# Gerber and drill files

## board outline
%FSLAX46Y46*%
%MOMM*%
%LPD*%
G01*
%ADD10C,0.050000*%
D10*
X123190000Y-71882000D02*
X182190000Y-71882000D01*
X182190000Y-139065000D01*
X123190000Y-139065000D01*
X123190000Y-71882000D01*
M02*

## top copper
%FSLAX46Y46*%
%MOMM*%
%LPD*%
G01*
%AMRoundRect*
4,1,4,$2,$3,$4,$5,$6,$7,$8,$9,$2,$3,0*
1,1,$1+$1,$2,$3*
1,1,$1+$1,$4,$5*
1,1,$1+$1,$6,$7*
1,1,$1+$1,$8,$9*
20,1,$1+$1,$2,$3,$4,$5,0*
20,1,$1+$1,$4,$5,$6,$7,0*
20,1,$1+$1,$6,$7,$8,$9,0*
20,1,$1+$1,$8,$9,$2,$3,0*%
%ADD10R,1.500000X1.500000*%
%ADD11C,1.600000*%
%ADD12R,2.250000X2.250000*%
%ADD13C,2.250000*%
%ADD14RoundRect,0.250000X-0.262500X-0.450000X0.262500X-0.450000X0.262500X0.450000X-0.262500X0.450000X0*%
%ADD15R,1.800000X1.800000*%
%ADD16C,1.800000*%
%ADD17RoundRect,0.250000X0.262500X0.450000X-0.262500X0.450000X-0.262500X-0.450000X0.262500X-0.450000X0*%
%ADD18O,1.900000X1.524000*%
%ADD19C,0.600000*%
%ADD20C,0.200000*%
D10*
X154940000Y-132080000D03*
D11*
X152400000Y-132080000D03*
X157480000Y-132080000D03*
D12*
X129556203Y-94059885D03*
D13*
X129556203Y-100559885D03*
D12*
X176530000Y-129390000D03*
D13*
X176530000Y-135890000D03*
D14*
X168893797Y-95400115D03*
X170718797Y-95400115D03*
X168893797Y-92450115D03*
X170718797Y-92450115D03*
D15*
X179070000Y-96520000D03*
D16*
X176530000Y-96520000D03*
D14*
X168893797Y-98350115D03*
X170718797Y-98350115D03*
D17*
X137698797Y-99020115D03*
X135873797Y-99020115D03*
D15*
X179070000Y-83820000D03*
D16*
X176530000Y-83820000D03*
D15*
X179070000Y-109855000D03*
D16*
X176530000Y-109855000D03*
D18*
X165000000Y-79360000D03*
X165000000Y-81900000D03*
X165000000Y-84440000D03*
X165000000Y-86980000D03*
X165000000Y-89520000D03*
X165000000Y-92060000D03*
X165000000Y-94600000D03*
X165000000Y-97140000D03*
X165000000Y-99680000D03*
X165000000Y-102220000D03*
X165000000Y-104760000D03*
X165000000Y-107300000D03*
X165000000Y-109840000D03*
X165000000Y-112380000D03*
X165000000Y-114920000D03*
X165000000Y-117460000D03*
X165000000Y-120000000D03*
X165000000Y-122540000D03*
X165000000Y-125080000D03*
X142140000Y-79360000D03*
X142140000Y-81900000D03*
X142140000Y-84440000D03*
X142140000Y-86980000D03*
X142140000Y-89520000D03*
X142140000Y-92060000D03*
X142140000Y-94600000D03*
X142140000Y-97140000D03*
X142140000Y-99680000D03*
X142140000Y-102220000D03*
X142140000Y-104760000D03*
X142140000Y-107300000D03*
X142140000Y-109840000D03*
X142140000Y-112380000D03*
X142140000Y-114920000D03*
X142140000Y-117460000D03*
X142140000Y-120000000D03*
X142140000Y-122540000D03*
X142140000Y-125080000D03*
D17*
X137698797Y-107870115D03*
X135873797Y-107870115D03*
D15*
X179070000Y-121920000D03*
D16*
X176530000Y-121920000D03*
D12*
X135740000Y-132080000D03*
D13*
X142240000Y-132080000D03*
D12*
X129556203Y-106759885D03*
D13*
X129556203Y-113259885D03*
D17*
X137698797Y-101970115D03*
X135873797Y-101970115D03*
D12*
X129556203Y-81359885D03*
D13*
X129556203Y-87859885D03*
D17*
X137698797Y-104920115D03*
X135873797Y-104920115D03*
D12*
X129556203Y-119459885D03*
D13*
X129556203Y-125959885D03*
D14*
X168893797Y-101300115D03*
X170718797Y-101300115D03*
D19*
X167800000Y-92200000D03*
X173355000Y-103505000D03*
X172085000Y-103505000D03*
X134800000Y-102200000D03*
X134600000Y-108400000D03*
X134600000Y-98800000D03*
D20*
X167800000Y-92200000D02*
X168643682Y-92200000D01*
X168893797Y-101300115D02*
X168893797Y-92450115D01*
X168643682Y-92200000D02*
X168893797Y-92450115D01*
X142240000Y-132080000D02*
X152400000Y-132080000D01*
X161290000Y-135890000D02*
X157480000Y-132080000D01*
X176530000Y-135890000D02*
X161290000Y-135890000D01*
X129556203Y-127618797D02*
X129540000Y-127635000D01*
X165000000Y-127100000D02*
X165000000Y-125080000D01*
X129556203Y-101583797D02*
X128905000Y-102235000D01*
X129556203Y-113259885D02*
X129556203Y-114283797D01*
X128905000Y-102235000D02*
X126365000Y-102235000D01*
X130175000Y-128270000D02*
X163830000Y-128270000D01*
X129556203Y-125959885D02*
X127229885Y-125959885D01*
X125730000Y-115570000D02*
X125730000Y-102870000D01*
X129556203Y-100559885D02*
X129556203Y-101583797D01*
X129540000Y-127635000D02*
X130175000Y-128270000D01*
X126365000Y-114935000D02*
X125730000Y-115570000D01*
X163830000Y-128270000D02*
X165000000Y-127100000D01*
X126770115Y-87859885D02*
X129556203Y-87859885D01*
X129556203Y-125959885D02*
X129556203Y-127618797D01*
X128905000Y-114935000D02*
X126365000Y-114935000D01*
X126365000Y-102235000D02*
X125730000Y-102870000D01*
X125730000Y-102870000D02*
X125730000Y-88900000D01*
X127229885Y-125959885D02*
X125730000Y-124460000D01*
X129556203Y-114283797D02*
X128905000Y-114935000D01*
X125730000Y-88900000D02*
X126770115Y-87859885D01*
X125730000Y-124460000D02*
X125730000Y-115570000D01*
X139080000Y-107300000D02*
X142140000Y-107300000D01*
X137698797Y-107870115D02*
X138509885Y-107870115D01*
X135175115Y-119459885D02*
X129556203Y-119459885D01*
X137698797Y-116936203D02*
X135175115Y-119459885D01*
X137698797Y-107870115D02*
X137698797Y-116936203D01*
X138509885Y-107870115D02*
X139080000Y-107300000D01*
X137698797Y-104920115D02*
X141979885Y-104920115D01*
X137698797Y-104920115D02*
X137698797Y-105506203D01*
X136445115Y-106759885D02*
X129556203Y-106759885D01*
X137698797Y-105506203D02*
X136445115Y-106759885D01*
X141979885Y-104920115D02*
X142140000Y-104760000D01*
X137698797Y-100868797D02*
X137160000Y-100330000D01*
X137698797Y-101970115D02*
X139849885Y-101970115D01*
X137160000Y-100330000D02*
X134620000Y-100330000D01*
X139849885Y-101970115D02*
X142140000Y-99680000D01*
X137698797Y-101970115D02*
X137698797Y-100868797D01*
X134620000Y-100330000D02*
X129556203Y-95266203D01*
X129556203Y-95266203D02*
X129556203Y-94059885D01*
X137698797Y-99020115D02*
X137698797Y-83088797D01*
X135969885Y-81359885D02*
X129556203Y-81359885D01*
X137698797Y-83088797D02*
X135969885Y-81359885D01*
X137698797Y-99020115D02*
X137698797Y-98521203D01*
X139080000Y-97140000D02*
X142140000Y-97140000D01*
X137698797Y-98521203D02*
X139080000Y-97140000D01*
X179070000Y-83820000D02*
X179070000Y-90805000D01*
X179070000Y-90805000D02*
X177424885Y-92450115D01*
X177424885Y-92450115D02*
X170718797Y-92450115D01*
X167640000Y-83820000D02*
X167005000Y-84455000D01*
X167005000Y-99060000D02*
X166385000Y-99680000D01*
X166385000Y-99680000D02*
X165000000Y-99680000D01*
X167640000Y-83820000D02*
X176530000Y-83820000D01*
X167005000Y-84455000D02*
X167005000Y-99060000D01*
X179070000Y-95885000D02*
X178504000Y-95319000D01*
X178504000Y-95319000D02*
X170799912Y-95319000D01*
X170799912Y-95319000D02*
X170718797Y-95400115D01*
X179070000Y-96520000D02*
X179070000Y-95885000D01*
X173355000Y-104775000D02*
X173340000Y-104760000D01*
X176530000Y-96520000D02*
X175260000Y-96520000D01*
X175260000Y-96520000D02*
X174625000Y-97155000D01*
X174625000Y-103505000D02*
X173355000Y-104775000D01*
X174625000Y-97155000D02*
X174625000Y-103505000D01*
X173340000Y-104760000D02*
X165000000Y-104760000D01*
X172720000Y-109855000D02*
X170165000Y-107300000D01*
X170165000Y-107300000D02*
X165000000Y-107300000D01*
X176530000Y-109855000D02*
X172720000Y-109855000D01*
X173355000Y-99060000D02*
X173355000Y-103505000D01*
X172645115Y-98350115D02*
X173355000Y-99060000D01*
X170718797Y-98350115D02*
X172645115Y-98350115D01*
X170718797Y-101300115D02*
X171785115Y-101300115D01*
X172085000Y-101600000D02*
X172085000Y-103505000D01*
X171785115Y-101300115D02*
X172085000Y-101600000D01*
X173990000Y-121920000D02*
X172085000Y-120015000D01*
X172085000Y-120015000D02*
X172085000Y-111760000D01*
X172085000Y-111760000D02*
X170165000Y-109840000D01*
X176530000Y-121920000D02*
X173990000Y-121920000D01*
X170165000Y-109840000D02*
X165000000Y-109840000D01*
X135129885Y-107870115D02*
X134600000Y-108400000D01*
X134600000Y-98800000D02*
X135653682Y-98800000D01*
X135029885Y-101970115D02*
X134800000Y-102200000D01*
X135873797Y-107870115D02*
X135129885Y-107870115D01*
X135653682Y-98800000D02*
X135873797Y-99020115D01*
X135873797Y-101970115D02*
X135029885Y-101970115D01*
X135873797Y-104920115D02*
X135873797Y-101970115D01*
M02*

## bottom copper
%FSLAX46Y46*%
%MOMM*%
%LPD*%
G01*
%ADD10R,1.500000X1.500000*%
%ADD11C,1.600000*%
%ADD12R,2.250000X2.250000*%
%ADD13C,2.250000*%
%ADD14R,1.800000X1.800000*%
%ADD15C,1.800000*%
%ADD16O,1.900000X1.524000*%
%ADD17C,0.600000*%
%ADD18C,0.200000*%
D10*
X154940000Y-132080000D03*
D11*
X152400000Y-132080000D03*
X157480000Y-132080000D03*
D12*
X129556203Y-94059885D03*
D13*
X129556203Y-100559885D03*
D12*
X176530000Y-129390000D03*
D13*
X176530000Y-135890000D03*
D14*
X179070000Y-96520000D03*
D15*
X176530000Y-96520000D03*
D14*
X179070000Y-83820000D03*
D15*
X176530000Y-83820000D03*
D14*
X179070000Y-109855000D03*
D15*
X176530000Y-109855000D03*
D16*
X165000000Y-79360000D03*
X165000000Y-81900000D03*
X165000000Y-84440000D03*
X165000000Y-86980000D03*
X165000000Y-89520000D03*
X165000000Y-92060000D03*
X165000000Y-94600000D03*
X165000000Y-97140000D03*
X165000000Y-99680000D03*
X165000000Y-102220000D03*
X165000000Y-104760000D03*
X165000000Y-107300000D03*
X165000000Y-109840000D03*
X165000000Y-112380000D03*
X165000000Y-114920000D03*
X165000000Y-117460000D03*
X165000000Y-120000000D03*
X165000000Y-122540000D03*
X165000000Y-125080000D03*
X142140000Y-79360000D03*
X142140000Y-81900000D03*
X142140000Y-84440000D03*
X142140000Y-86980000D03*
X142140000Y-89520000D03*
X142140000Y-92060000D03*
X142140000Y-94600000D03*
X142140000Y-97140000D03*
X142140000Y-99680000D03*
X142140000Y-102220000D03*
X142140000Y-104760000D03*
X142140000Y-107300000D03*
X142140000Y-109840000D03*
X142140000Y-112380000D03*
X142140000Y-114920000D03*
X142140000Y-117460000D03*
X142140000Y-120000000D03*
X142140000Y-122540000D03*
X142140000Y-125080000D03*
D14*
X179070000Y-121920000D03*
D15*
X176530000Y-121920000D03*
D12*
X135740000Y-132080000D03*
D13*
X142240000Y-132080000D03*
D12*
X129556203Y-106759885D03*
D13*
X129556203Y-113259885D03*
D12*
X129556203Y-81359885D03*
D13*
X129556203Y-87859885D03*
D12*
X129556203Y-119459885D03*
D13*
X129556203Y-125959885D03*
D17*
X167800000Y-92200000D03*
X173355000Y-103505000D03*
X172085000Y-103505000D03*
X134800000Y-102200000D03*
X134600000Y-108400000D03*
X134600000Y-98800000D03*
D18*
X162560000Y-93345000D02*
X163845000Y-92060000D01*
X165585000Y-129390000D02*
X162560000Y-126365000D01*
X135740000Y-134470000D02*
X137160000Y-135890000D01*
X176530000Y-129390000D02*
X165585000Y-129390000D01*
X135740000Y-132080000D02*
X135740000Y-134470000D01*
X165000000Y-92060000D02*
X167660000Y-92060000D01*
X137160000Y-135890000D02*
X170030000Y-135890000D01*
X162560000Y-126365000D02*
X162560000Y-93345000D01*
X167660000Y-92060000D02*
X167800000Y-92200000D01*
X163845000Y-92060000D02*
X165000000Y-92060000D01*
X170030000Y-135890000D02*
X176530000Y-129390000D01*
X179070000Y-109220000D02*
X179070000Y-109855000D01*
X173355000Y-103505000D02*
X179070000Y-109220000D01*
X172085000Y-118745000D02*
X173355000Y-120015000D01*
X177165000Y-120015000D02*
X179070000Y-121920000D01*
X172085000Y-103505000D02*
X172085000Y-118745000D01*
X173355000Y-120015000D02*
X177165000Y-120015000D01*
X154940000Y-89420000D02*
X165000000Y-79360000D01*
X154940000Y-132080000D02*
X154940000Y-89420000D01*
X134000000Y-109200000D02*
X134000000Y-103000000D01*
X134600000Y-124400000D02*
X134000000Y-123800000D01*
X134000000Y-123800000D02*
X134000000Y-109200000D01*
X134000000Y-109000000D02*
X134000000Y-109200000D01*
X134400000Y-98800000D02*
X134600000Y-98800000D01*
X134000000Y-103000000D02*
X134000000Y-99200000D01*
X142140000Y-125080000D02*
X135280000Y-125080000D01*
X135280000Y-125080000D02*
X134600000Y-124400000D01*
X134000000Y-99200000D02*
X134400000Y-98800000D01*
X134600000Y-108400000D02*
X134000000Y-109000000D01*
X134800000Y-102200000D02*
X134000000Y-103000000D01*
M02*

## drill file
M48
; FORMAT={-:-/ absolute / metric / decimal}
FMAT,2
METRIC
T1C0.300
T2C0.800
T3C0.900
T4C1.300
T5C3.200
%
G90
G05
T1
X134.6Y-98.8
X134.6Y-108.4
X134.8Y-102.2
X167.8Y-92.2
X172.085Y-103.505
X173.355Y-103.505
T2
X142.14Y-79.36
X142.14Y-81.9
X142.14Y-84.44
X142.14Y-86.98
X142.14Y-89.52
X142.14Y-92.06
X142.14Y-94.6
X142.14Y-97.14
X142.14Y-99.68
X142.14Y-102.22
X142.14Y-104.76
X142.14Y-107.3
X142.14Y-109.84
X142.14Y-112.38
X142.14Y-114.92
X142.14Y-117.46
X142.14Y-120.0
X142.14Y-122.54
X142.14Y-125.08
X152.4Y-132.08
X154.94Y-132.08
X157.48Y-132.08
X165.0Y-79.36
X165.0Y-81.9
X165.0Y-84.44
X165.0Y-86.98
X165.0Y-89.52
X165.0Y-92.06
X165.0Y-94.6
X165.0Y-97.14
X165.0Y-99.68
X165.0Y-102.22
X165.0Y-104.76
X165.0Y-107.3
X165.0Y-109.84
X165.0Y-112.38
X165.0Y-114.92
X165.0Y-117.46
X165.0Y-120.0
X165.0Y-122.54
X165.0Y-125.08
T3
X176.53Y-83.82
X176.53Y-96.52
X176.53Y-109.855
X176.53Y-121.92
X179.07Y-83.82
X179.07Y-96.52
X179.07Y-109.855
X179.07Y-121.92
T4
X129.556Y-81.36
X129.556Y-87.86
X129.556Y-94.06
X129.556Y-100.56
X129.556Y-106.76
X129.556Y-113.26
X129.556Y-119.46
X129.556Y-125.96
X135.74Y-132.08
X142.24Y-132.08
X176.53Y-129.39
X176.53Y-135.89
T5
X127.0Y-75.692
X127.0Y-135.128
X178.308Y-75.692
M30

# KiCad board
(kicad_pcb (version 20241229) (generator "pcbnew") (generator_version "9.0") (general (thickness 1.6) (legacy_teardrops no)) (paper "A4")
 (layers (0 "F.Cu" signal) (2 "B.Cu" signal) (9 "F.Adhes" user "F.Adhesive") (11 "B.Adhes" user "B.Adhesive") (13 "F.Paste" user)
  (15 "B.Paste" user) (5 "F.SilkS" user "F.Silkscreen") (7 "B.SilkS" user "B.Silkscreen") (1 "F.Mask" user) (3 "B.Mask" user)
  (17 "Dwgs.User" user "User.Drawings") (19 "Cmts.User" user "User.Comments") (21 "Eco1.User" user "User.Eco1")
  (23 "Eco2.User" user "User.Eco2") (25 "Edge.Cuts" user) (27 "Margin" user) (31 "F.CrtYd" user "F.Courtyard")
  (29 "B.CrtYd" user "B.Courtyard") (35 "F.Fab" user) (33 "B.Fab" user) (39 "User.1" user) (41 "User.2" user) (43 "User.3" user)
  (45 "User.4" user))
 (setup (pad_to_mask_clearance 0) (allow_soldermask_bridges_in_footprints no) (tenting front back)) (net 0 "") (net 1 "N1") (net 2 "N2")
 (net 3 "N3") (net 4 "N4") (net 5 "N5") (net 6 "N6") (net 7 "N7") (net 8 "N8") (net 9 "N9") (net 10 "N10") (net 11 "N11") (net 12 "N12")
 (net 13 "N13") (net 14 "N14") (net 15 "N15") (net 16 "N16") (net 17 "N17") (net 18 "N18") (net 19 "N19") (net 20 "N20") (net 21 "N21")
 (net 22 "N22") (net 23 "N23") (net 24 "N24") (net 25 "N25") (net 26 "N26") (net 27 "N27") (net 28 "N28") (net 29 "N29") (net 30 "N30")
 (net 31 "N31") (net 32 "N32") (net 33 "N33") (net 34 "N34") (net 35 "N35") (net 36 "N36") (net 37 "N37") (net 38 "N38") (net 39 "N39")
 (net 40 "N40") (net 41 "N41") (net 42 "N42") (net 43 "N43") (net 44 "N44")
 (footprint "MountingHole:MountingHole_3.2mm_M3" (layer "F.Cu") (at 178.308 75.692)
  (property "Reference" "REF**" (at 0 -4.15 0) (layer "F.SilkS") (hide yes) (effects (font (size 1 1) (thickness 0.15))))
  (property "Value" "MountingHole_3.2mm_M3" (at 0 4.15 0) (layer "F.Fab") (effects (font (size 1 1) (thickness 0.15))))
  (pad "" np_thru_hole circle (at 0 0) (size 3.2 3.2) (drill 3.2) (layers "*.Cu" "*.Mask")))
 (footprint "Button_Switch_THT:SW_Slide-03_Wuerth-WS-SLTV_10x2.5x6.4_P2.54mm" (layer "F.Cu") (at 154.94 132.08)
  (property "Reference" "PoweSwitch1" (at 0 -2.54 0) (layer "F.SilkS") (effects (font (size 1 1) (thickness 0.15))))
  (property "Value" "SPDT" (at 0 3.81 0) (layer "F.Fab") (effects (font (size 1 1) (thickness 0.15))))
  (pad "1" thru_hole rect (at 0 0) (size 1.5 1.5) (drill 0.8) (layers "*.Cu" "*.Mask") (remove_unused_layers no) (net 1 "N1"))
  (pad "2" thru_hole circle (at -2.54 0) (size 1.6 1.6) (drill 0.8) (layers "*.Cu" "*.Mask") (remove_unused_layers no) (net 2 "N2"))
  (pad "3" thru_hole circle (at 2.54 0) (size 1.6 1.6) (drill 0.8) (layers "*.Cu" "*.Mask") (remove_unused_layers no) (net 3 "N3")))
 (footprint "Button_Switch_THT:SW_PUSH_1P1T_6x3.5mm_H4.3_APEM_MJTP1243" (layer "F.Cu") (at 129.556203 94.059885 -90)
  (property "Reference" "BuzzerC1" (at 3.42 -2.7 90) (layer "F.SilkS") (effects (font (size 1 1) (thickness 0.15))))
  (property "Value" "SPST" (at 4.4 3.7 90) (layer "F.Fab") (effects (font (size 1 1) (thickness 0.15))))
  (pad "1" thru_hole rect (at 0 0) (size 2.25 2.25) (drill 1.3) (layers "*.Cu" "*.Mask") (remove_unused_layers no) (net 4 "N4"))
  (pad "2" thru_hole circle (at 6.5 0) (size 2.25 2.25) (drill 1.3) (layers "*.Cu" "*.Mask") (remove_unused_layers no) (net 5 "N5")))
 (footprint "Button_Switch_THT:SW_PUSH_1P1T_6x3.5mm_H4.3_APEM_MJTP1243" (layer "F.Cu") (at 176.53 129.39 -90)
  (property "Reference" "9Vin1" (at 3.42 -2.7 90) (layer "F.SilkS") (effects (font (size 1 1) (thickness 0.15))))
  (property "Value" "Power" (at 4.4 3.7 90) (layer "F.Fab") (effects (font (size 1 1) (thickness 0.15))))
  (pad "1" thru_hole rect (at 0 0) (size 2.25 2.25) (drill 1.3) (layers "*.Cu" "*.Mask") (remove_unused_layers no) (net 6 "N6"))
  (pad "2" thru_hole circle (at 6.5 0) (size 2.25 2.25) (drill 1.3) (layers "*.Cu" "*.Mask") (remove_unused_layers no) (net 3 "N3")))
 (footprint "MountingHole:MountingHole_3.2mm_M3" (layer "F.Cu") (at 127 135.128)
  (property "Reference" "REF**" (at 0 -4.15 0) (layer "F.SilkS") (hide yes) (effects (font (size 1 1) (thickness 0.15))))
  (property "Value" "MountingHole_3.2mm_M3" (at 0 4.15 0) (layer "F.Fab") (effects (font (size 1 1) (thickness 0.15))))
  (pad "" np_thru_hole circle (at 0 0) (size 3.2 3.2) (drill 3.2) (layers "*.Cu" "*.Mask")))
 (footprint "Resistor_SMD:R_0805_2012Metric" (layer "F.Cu") (at 169.806297 95.400115)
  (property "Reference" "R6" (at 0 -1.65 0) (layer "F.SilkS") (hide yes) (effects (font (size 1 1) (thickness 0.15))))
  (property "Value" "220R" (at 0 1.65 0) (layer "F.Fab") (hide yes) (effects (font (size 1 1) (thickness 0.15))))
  (pad "1" smd roundrect (at -0.9125 0) (size 1.025 1.4) (layers "F.Cu" "F.Mask" "F.Paste") (roundrect_rratio 0.243902) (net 6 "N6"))
  (pad "2" smd roundrect (at 0.9125 0) (size 1.025 1.4) (layers "F.Cu" "F.Mask" "F.Paste") (roundrect_rratio 0.243902) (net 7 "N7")))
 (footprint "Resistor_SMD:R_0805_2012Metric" (layer "F.Cu") (at 169.806297 92.450115)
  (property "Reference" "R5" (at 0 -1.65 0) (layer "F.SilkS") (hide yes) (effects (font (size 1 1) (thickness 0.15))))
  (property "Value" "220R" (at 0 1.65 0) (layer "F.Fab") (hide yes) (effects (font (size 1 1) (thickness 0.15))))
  (pad "1" smd roundrect (at -0.9125 0) (size 1.025 1.4) (layers "F.Cu" "F.Mask" "F.Paste") (roundrect_rratio 0.243902) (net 6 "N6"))
  (pad "2" smd roundrect (at 0.9125 0) (size 1.025 1.4) (layers "F.Cu" "F.Mask" "F.Paste") (roundrect_rratio 0.243902) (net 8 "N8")))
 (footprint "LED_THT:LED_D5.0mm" (layer "F.Cu") (at 179.07 96.52 180)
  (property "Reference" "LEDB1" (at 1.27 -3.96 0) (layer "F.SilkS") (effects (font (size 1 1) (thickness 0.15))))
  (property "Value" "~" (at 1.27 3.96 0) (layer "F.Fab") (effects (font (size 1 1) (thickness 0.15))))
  (pad "1" thru_hole rect (at 0 0 180) (size 1.8 1.8) (drill 0.9) (layers "*.Cu" "*.Mask") (remove_unused_layers no) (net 7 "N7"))
  (pad "2" thru_hole circle (at 2.54 0 180) (size 1.8 1.8) (drill 0.9) (layers "*.Cu" "*.Mask") (remove_unused_layers no) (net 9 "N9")))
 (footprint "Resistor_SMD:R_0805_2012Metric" (layer "F.Cu") (at 169.806297 98.350115)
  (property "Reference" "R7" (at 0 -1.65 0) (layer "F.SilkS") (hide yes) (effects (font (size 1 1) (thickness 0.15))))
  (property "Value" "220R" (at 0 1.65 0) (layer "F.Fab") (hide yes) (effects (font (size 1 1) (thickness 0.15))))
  (pad "1" smd roundrect (at -0.9125 0) (size 1.025 1.4) (layers "F.Cu" "F.Mask" "F.Paste") (roundrect_rratio 0.243902) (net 6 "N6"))
  (pad "2" smd roundrect (at 0.9125 0) (size 1.025 1.4) (layers "F.Cu" "F.Mask" "F.Paste") (roundrect_rratio 0.243902) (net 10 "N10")))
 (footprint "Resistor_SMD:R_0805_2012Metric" (layer "F.Cu") (at 136.786297 99.020115 180)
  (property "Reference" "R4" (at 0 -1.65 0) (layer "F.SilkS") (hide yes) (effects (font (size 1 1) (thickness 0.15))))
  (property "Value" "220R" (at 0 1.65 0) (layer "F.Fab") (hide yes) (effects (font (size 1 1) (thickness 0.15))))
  (pad "1" smd roundrect (at -0.9125 0 180) (size 1.025 1.4) (layers "F.Cu" "F.Mask" "F.Paste") (roundrect_rratio 0.243902) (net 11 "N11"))
  (pad "2" smd roundrect (at 0.9125 0 180) (size 1.025 1.4) (layers "F.Cu" "F.Mask" "F.Paste") (roundrect_rratio 0.243902) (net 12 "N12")))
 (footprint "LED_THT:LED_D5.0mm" (layer "F.Cu") (at 179.07 83.82 180)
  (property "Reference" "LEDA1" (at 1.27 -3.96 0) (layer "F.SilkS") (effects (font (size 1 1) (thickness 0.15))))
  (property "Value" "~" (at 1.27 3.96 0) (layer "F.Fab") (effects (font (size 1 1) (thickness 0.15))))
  (pad "1" thru_hole rect (at 0 0 180) (size 1.8 1.8) (drill 0.9) (layers "*.Cu" "*.Mask") (remove_unused_layers no) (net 8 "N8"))
  (pad "2" thru_hole circle (at 2.54 0 180) (size 1.8 1.8) (drill 0.9) (layers "*.Cu" "*.Mask") (remove_unused_layers no) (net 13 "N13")))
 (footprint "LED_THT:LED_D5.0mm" (layer "F.Cu") (at 179.07 109.855 180)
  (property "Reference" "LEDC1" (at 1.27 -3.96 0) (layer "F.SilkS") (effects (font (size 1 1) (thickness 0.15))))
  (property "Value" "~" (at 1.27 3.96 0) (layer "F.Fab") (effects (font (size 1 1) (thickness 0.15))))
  (pad "1" thru_hole rect (at 0 0 180) (size 1.8 1.8) (drill 0.9) (layers "*.Cu" "*.Mask") (remove_unused_layers no) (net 10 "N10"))
  (pad "2" thru_hole circle (at 2.54 0 180) (size 1.8 1.8) (drill 0.9) (layers "*.Cu" "*.Mask") (remove_unused_layers no) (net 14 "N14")))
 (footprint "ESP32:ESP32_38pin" (layer "F.Cu") (at 153.456183 102.385111 180)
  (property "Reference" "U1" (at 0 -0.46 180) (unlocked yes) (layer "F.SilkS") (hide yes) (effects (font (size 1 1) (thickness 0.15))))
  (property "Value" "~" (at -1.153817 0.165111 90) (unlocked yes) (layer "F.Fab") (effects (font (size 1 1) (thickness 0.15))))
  (pad "1" thru_hole oval (at -11.543817 23.025111 90) (size 1.524 1.9) (drill 0.8) (layers "*.Cu" "*.Mask") (remove_unused_layers no)
   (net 1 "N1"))
  (pad "2" thru_hole oval (at -11.543817 20.485111 90) (size 1.524 1.9) (drill 0.8) (layers "*.Cu" "*.Mask") (remove_unused_layers no)
   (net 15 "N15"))
  (pad "3" thru_hole oval (at -11.543817 17.945111 90) (size 1.524 1.9) (drill 0.8) (layers "*.Cu" "*.Mask") (remove_unused_layers no)
   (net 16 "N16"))
  (pad "4" thru_hole oval (at -11.543817 15.405111 90) (size 1.524 1.9) (drill 0.8) (layers "*.Cu" "*.Mask") (remove_unused_layers no)
   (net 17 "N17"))
  (pad "5" thru_hole oval (at -11.543817 12.865111 90) (size 1.524 1.9) (drill 0.8) (layers "*.Cu" "*.Mask") (remove_unused_layers no)
   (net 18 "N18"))
  (pad "6" thru_hole oval (at -11.543817 10.325111 90) (size 1.524 1.9) (drill 0.8) (layers "*.Cu" "*.Mask") (remove_unused_layers no)
   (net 6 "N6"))
  (pad "7" thru_hole oval (at -11.543817 7.785111 90) (size 1.524 1.9) (drill 0.8) (layers "*.Cu" "*.Mask") (remove_unused_layers no)
   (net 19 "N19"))
  (pad "8" thru_hole oval (at -11.543817 5.245111 90) (size 1.524 1.9) (drill 0.8) (layers "*.Cu" "*.Mask") (remove_unused_layers no)
   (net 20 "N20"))
  (pad "9" thru_hole oval (at -11.543817 2.705111 90) (size 1.524 1.9) (drill 0.8) (layers "*.Cu" "*.Mask") (remove_unused_layers no)
   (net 13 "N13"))
  (pad "10" thru_hole oval (at -11.543817 0.165111 90) (size 1.524 1.9) (drill 0.8) (layers "*.Cu" "*.Mask") (remove_unused_layers no)
   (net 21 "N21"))
  (pad "11" thru_hole oval (at -11.543817 -2.374889 90) (size 1.524 1.9) (drill 0.8) (layers "*.Cu" "*.Mask") (remove_unused_layers no)
   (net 9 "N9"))
  (pad "12" thru_hole oval (at -11.543817 -4.914889 90) (size 1.524 1.9) (drill 0.8) (layers "*.Cu" "*.Mask") (remove_unused_layers no)
   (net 14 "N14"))
  (pad "13" thru_hole oval (at -11.543817 -7.454889 90) (size 1.524 1.9) (drill 0.8) (layers "*.Cu" "*.Mask") (remove_unused_layers no)
   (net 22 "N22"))
  (pad "14" thru_hole oval (at -11.543817 -9.994889 90) (size 1.524 1.9) (drill 0.8) (layers "*.Cu" "*.Mask") (remove_unused_layers no)
   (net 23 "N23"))
  (pad "15" thru_hole oval (at -11.543817 -12.534889 90) (size 1.524 1.9) (drill 0.8) (layers "*.Cu" "*.Mask") (remove_unused_layers no)
   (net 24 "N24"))
  (pad "16" thru_hole oval (at -11.543817 -15.074889 90) (size 1.524 1.9) (drill 0.8) (layers "*.Cu" "*.Mask") (remove_unused_layers no)
   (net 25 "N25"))
  (pad "17" thru_hole oval (at -11.543817 -17.614889 90) (size 1.524 1.9) (drill 0.8) (layers "*.Cu" "*.Mask") (remove_unused_layers no)
   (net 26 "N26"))
  (pad "18" thru_hole oval (at -11.543817 -20.154889 90) (size 1.524 1.9) (drill 0.8) (layers "*.Cu" "*.Mask") (remove_unused_layers no)
   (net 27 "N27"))
  (pad "19" thru_hole oval (at -11.543817 -22.694889 90) (size 1.524 1.9) (drill 0.8) (layers "*.Cu" "*.Mask") (remove_unused_layers no)
   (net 5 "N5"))
  (pad "20" thru_hole oval (at 11.316183 23.025111 90) (size 1.524 1.9) (drill 0.8) (layers "*.Cu" "*.Mask") (remove_unused_layers no)
   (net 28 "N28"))
  (pad "21" thru_hole oval (at 11.316183 20.485111 90) (size 1.524 1.9) (drill 0.8) (layers "*.Cu" "*.Mask") (remove_unused_layers no)
   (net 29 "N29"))
  (pad "22" thru_hole oval (at 11.316183 17.945111 90) (size 1.524 1.9) (drill 0.8) (layers "*.Cu" "*.Mask") (remove_unused_layers no)
   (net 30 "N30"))
  (pad "23" thru_hole oval (at 11.316183 15.405111 90) (size 1.524 1.9) (drill 0.8) (layers "*.Cu" "*.Mask") (remove_unused_layers no)
   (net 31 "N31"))
  (pad "24" thru_hole oval (at 11.316183 12.865111 90) (size 1.524 1.9) (drill 0.8) (layers "*.Cu" "*.Mask") (remove_unused_layers no)
   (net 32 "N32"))
  (pad "25" thru_hole oval (at 11.316183 10.325111 90) (size 1.524 1.9) (drill 0.8) (layers "*.Cu" "*.Mask") (remove_unused_layers no)
   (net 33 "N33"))
  (pad "26" thru_hole oval (at 11.316183 7.785111 90) (size 1.524 1.9) (drill 0.8) (layers "*.Cu" "*.Mask") (remove_unused_layers no)
   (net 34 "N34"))
  (pad "27" thru_hole oval (at 11.316183 5.245111 90) (size 1.524 1.9) (drill 0.8) (layers "*.Cu" "*.Mask") (remove_unused_layers no)
   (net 11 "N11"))
  (pad "28" thru_hole oval (at 11.316183 2.705111 90) (size 1.524 1.9) (drill 0.8) (layers "*.Cu" "*.Mask") (remove_unused_layers no)
   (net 4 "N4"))
  (pad "29" thru_hole oval (at 11.316183 0.165111 90) (size 1.524 1.9) (drill 0.8) (layers "*.Cu" "*.Mask") (remove_unused_layers no)
   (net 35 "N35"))
  (pad "30" thru_hole oval (at 11.316183 -2.374889 90) (size 1.524 1.9) (drill 0.8) (layers "*.Cu" "*.Mask") (remove_unused_layers no)
   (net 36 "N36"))
  (pad "31" thru_hole oval (at 11.316183 -4.914889 90) (size 1.524 1.9) (drill 0.8) (layers "*.Cu" "*.Mask") (remove_unused_layers no)
   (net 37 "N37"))
  (pad "32" thru_hole oval (at 11.316183 -7.454889 90) (size 1.524 1.9) (drill 0.8) (layers "*.Cu" "*.Mask") (remove_unused_layers no)
   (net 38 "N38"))
  (pad "33" thru_hole oval (at 11.316183 -9.994889 90) (size 1.524 1.9) (drill 0.8) (layers "*.Cu" "*.Mask") (remove_unused_layers no)
   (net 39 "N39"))
  (pad "34" thru_hole oval (at 11.316183 -12.534889 90) (size 1.524 1.9) (drill 0.8) (layers "*.Cu" "*.Mask") (remove_unused_layers no)
   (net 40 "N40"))
  (pad "35" thru_hole oval (at 11.316183 -15.074889 90) (size 1.524 1.9) (drill 0.8) (layers "*.Cu" "*.Mask") (remove_unused_layers no)
   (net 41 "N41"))
  (pad "36" thru_hole oval (at 11.316183 -17.614889 90) (size 1.524 1.9) (drill 0.8) (layers "*.Cu" "*.Mask") (remove_unused_layers no)
   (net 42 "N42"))
  (pad "37" thru_hole oval (at 11.316183 -20.154889 90) (size 1.524 1.9) (drill 0.8) (layers "*.Cu" "*.Mask") (remove_unused_layers no)
   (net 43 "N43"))
  (pad "38" thru_hole oval (at 11.316183 -22.694889 90) (size 1.524 1.9) (drill 0.8) (layers "*.Cu" "*.Mask") (remove_unused_layers no)
   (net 12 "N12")))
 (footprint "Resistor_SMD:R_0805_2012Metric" (layer "F.Cu") (at 136.786297 107.870115 180)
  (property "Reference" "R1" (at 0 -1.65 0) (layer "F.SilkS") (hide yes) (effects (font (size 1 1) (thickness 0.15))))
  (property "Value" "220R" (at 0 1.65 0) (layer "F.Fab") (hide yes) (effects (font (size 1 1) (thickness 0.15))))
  (pad "1" smd roundrect (at -0.9125 0 180) (size 1.025 1.4) (layers "F.Cu" "F.Mask" "F.Paste") (roundrect_rratio 0.243902) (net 37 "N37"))
  (pad "2" smd roundrect (at 0.9125 0 180) (size 1.025 1.4) (layers "F.Cu" "F.Mask" "F.Paste") (roundrect_rratio 0.243902) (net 12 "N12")))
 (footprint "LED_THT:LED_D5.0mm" (layer "F.Cu") (at 179.07 121.92 180)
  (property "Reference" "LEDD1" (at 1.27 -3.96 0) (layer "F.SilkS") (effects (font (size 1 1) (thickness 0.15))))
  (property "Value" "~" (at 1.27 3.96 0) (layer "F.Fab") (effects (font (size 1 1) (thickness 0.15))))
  (pad "1" thru_hole rect (at 0 0 180) (size 1.8 1.8) (drill 0.9) (layers "*.Cu" "*.Mask") (remove_unused_layers no) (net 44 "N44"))
  (pad "2" thru_hole circle (at 2.54 0 180) (size 1.8 1.8) (drill 0.9) (layers "*.Cu" "*.Mask") (remove_unused_layers no) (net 22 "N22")))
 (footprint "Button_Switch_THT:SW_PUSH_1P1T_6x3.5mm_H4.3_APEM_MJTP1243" (layer "F.Cu") (at 135.74 132.08)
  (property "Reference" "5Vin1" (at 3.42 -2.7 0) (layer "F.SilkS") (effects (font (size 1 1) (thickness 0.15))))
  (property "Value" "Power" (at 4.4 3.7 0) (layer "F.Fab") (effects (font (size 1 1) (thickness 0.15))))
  (pad "1" thru_hole rect (at 0 0 90) (size 2.25 2.25) (drill 1.3) (layers "*.Cu" "*.Mask") (remove_unused_layers no) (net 6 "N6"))
  (pad "2" thru_hole circle (at 6.5 0 90) (size 2.25 2.25) (drill 1.3) (layers "*.Cu" "*.Mask") (remove_unused_layers no) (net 2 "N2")))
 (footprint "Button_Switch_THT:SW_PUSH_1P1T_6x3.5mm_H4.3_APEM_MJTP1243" (layer "F.Cu") (at 129.556203 106.759885 -90)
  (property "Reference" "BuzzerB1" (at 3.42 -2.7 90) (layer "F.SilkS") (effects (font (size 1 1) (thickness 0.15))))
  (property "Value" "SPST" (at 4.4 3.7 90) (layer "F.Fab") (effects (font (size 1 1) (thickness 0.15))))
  (pad "1" thru_hole rect (at 0 0) (size 2.25 2.25) (drill 1.3) (layers "*.Cu" "*.Mask") (remove_unused_layers no) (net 36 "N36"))
  (pad "2" thru_hole circle (at 6.5 0) (size 2.25 2.25) (drill 1.3) (layers "*.Cu" "*.Mask") (remove_unused_layers no) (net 5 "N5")))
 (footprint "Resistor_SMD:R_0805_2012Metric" (layer "F.Cu") (at 136.786297 101.970115 180)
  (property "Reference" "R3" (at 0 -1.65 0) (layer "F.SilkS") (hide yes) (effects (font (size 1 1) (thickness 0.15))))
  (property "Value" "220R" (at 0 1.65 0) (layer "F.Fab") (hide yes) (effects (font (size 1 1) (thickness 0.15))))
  (pad "1" smd roundrect (at -0.9125 0 180) (size 1.025 1.4) (layers "F.Cu" "F.Mask" "F.Paste") (roundrect_rratio 0.243902) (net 4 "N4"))
  (pad "2" smd roundrect (at 0.9125 0 180) (size 1.025 1.4) (layers "F.Cu" "F.Mask" "F.Paste") (roundrect_rratio 0.243902) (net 12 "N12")))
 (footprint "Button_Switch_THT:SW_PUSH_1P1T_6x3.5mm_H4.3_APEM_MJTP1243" (layer "F.Cu") (at 129.556203 81.359885 -90)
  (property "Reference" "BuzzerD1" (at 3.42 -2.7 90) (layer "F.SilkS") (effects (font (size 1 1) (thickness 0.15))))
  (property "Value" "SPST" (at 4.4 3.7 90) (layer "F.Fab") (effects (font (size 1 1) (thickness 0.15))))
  (pad "1" thru_hole rect (at 0 0) (size 2.25 2.25) (drill 1.3) (layers "*.Cu" "*.Mask") (remove_unused_layers no) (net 11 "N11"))
  (pad "2" thru_hole circle (at 6.5 0) (size 2.25 2.25) (drill 1.3) (layers "*.Cu" "*.Mask") (remove_unused_layers no) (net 5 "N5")))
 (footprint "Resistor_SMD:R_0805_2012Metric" (layer "F.Cu") (at 136.786297 104.920115 180)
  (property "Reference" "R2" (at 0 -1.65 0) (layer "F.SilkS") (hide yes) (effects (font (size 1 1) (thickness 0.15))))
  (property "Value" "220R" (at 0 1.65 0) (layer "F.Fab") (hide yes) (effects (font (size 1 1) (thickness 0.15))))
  (pad "1" smd roundrect (at -0.9125 0 180) (size 1.025 1.4) (layers "F.Cu" "F.Mask" "F.Paste") (roundrect_rratio 0.243902) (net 36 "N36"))
  (pad "2" smd roundrect (at 0.9125 0 180) (size 1.025 1.4) (layers "F.Cu" "F.Mask" "F.Paste") (roundrect_rratio 0.243902) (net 12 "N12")))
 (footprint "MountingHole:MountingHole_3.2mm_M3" (layer "F.Cu") (at 127 75.692)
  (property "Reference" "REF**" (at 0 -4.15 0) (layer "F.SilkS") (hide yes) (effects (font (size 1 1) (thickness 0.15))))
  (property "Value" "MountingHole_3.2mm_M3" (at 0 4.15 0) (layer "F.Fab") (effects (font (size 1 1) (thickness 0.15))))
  (pad "" np_thru_hole circle (at 0 0) (size 3.2 3.2) (drill 3.2) (layers "*.Cu" "*.Mask")))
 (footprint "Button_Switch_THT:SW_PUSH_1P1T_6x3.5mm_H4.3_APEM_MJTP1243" (layer "F.Cu") (at 129.556203 119.459885 -90)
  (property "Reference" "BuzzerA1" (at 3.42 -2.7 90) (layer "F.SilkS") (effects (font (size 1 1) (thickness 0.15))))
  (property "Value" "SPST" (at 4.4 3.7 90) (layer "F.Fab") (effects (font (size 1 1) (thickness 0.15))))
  (pad "1" thru_hole rect (at 0 0) (size 2.25 2.25) (drill 1.3) (layers "*.Cu" "*.Mask") (remove_unused_layers no) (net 37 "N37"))
  (pad "2" thru_hole circle (at 6.5 0) (size 2.25 2.25) (drill 1.3) (layers "*.Cu" "*.Mask") (remove_unused_layers no) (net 5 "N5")))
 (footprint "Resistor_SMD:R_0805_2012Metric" (layer "F.Cu") (at 169.806297 101.300115)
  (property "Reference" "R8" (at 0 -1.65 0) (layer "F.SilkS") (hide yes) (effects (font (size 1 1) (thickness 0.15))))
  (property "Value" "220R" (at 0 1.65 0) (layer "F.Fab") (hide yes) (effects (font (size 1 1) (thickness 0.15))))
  (pad "1" smd roundrect (at -0.9125 0) (size 1.025 1.4) (layers "F.Cu" "F.Mask" "F.Paste") (roundrect_rratio 0.243902) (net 6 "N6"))
  (pad "2" smd roundrect (at 0.9125 0) (size 1.025 1.4) (layers "F.Cu" "F.Mask" "F.Paste") (roundrect_rratio 0.243902) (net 44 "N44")))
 (gr_rect (start 123.19 71.882) (end 182.19 139.065) (stroke (width 0.05) (type solid)) (fill no) (layer "Edge.Cuts"))
 (segment (start 167.8 92.2) (end 168.643682 92.2) (width 0.2) (layer "F.Cu") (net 6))
 (segment (start 168.893797 101.300115) (end 168.893797 92.450115) (width 0.2) (layer "F.Cu") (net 6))
 (segment (start 168.643682 92.2) (end 168.893797 92.450115) (width 0.2) (layer "F.Cu") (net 6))
 (via (at 167.8 92.2) (size 0.6) (drill 0.3) (layers "F.Cu" "B.Cu") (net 6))
 (segment (start 162.56 93.345) (end 163.845 92.06) (width 0.2) (layer "B.Cu") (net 6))
 (segment (start 165.585 129.39) (end 162.56 126.365) (width 0.2) (layer "B.Cu") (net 6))
 (segment (start 135.74 134.47) (end 137.16 135.89) (width 0.2) (layer "B.Cu") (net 6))
 (segment (start 176.53 129.39) (end 165.585 129.39) (width 0.2) (layer "B.Cu") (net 6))
 (segment (start 135.74 132.08) (end 135.74 134.47) (width 0.2) (layer "B.Cu") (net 6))
 (segment (start 165 92.06) (end 167.66 92.06) (width 0.2) (layer "B.Cu") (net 6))
 (segment (start 137.16 135.89) (end 170.03 135.89) (width 0.2) (layer "B.Cu") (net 6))
 (segment (start 162.56 126.365) (end 162.56 93.345) (width 0.2) (layer "B.Cu") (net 6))
 (segment (start 167.66 92.06) (end 167.8 92.2) (width 0.2) (layer "B.Cu") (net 6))
 (segment (start 163.845 92.06) (end 165 92.06) (width 0.2) (layer "B.Cu") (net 6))
 (segment (start 170.03 135.89) (end 176.53 129.39) (width 0.2) (layer "B.Cu") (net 6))
 (segment (start 142.24 132.08) (end 152.4 132.08) (width 0.2) (layer "F.Cu") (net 2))
 (segment (start 161.29 135.89) (end 157.48 132.08) (width 0.2) (layer "F.Cu") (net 3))
 (segment (start 176.53 135.89) (end 161.29 135.89) (width 0.2) (layer "F.Cu") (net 3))
 (segment (start 129.556203 127.618797) (end 129.54 127.635) (width 0.2) (layer "F.Cu") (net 5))
 (segment (start 165 127.1) (end 165 125.08) (width 0.2) (layer "F.Cu") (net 5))
 (segment (start 129.556203 101.583797) (end 128.905 102.235) (width 0.2) (layer "F.Cu") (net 5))
 (segment (start 129.556203 113.259885) (end 129.556203 114.283797) (width 0.2) (layer "F.Cu") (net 5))
 (segment (start 128.905 102.235) (end 126.365 102.235) (width 0.2) (layer "F.Cu") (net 5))
 (segment (start 130.175 128.27) (end 163.83 128.27) (width 0.2) (layer "F.Cu") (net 5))
 (segment (start 129.556203 125.959885) (end 127.229885 125.959885) (width 0.2) (layer "F.Cu") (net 5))
 (segment (start 125.73 115.57) (end 125.73 102.87) (width 0.2) (layer "F.Cu") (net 5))
 (segment (start 129.556203 100.559885) (end 129.556203 101.583797) (width 0.2) (layer "F.Cu") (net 5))
 (segment (start 129.54 127.635) (end 130.175 128.27) (width 0.2) (layer "F.Cu") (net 5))
 (segment (start 126.365 114.935) (end 125.73 115.57) (width 0.2) (layer "F.Cu") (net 5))
 (segment (start 163.83 128.27) (end 165 127.1) (width 0.2) (layer "F.Cu") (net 5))
 (segment (start 126.770115 87.859885) (end 129.556203 87.859885) (width 0.2) (layer "F.Cu") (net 5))
 (segment (start 129.556203 125.959885) (end 129.556203 127.618797) (width 0.2) (layer "F.Cu") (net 5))
 (segment (start 128.905 114.935) (end 126.365 114.935) (width 0.2) (layer "F.Cu") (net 5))
 (segment (start 126.365 102.235) (end 125.73 102.87) (width 0.2) (layer "F.Cu") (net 5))
 (segment (start 125.73 102.87) (end 125.73 88.9) (width 0.2) (layer "F.Cu") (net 5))
 (segment (start 127.229885 125.959885) (end 125.73 124.46) (width 0.2) (layer "F.Cu") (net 5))
 (segment (start 129.556203 114.283797) (end 128.905 114.935) (width 0.2) (layer "F.Cu") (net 5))
 (segment (start 125.73 88.9) (end 126.770115 87.859885) (width 0.2) (layer "F.Cu") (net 5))
 (segment (start 125.73 124.46) (end 125.73 115.57) (width 0.2) (layer "F.Cu") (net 5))
 (segment (start 139.08 107.3) (end 142.14 107.3) (width 0.2) (layer "F.Cu") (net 37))
 (segment (start 137.698797 107.870115) (end 138.509885 107.870115) (width 0.2) (layer "F.Cu") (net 37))
 (segment (start 135.175115 119.459885) (end 129.556203 119.459885) (width 0.2) (layer "F.Cu") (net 37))
 (segment (start 137.698797 116.936203) (end 135.175115 119.459885) (width 0.2) (layer "F.Cu") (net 37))
 (segment (start 137.698797 107.870115) (end 137.698797 116.936203) (width 0.2) (layer "F.Cu") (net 37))
 (segment (start 138.509885 107.870115) (end 139.08 107.3) (width 0.2) (layer "F.Cu") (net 37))
 (segment (start 137.698797 104.920115) (end 141.979885 104.920115) (width 0.2) (layer "F.Cu") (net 36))
 (segment (start 137.698797 104.920115) (end 137.698797 105.506203) (width 0.2) (layer "F.Cu") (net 36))
 (segment (start 136.445115 106.759885) (end 129.556203 106.759885) (width 0.2) (layer "F.Cu") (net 36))
 (segment (start 137.698797 105.506203) (end 136.445115 106.759885) (width 0.2) (layer "F.Cu") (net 36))
 (segment (start 141.979885 104.920115) (end 142.14 104.76) (width 0.2) (layer "F.Cu") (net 36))
 (segment (start 137.698797 100.868797) (end 137.16 100.33) (width 0.2) (layer "F.Cu") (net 4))
 (segment (start 137.698797 101.970115) (end 139.849885 101.970115) (width 0.2) (layer "F.Cu") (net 4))
 (segment (start 137.16 100.33) (end 134.62 100.33) (width 0.2) (layer "F.Cu") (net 4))
 (segment (start 139.849885 101.970115) (end 142.14 99.68) (width 0.2) (layer "F.Cu") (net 4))
 (segment (start 137.698797 101.970115) (end 137.698797 100.868797) (width 0.2) (layer "F.Cu") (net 4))
 (segment (start 134.62 100.33) (end 129.556203 95.266203) (width 0.2) (layer "F.Cu") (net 4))
 (segment (start 129.556203 95.266203) (end 129.556203 94.059885) (width 0.2) (layer "F.Cu") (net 4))
 (segment (start 137.698797 99.020115) (end 137.698797 83.088797) (width 0.2) (layer "F.Cu") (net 11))
 (segment (start 135.969885 81.359885) (end 129.556203 81.359885) (width 0.2) (layer "F.Cu") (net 11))
 (segment (start 137.698797 83.088797) (end 135.969885 81.359885) (width 0.2) (layer "F.Cu") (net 11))
 (segment (start 137.698797 99.020115) (end 137.698797 98.521203) (width 0.2) (layer "F.Cu") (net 11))
 (segment (start 139.08 97.14) (end 142.14 97.14) (width 0.2) (layer "F.Cu") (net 11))
 (segment (start 137.698797 98.521203) (end 139.08 97.14) (width 0.2) (layer "F.Cu") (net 11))
 (segment (start 179.07 83.82) (end 179.07 90.805) (width 0.2) (layer "F.Cu") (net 8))
 (segment (start 179.07 90.805) (end 177.424885 92.450115) (width 0.2) (layer "F.Cu") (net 8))
 (segment (start 177.424885 92.450115) (end 170.718797 92.450115) (width 0.2) (layer "F.Cu") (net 8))
 (segment (start 167.64 83.82) (end 167.005 84.455) (width 0.2) (layer "F.Cu") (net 13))
 (segment (start 167.005 99.06) (end 166.385 99.68) (width 0.2) (layer "F.Cu") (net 13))
 (segment (start 166.385 99.68) (end 165 99.68) (width 0.2) (layer "F.Cu") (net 13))
 (segment (start 167.64 83.82) (end 176.53 83.82) (width 0.2) (layer "F.Cu") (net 13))
 (segment (start 167.005 84.455) (end 167.005 99.06) (width 0.2) (layer "F.Cu") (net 13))
 (segment (start 179.07 95.885) (end 178.504 95.319) (width 0.2) (layer "F.Cu") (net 7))
 (segment (start 178.504 95.319) (end 170.799912 95.319) (width 0.2) (layer "F.Cu") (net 7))
 (segment (start 170.799912 95.319) (end 170.718797 95.400115) (width 0.2) (layer "F.Cu") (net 7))
 (segment (start 179.07 96.52) (end 179.07 95.885) (width 0.2) (layer "F.Cu") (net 7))
 (segment (start 173.355 104.775) (end 173.34 104.76) (width 0.2) (layer "F.Cu") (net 9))
 (segment (start 176.53 96.52) (end 175.26 96.52) (width 0.2) (layer "F.Cu") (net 9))
 (segment (start 175.26 96.52) (end 174.625 97.155) (width 0.2) (layer "F.Cu") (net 9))
 (segment (start 174.625 103.505) (end 173.355 104.775) (width 0.2) (layer "F.Cu") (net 9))
 (segment (start 174.625 97.155) (end 174.625 103.505) (width 0.2) (layer "F.Cu") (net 9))
 (segment (start 173.34 104.76) (end 165 104.76) (width 0.2) (layer "F.Cu") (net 9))
 (segment (start 172.72 109.855) (end 170.165 107.3) (width 0.2) (layer "F.Cu") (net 14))
 (segment (start 170.165 107.3) (end 165 107.3) (width 0.2) (layer "F.Cu") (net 14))
 (segment (start 176.53 109.855) (end 172.72 109.855) (width 0.2) (layer "F.Cu") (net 14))
 (segment (start 173.355 99.06) (end 173.355 103.505) (width 0.2) (layer "F.Cu") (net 10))
 (segment (start 172.645115 98.350115) (end 173.355 99.06) (width 0.2) (layer "F.Cu") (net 10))
 (segment (start 170.718797 98.350115) (end 172.645115 98.350115) (width 0.2) (layer "F.Cu") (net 10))
 (via (at 173.355 103.505) (size 0.6) (drill 0.3) (layers "F.Cu" "B.Cu") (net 10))
 (segment (start 179.07 109.22) (end 179.07 109.855) (width 0.2) (layer "B.Cu") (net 10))
 (segment (start 173.355 103.505) (end 179.07 109.22) (width 0.2) (layer "B.Cu") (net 10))
 (segment (start 170.718797 101.300115) (end 171.785115 101.300115) (width 0.2) (layer "F.Cu") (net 44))
 (segment (start 172.085 101.6) (end 172.085 103.505) (width 0.2) (layer "F.Cu") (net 44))
 (segment (start 171.785115 101.300115) (end 172.085 101.6) (width 0.2) (layer "F.Cu") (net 44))
 (via (at 172.085 103.505) (size 0.6) (drill 0.3) (layers "F.Cu" "B.Cu") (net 44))
 (segment (start 172.085 118.745) (end 173.355 120.015) (width 0.2) (layer "B.Cu") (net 44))
 (segment (start 177.165 120.015) (end 179.07 121.92) (width 0.2) (layer "B.Cu") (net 44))
 (segment (start 172.085 103.505) (end 172.085 118.745) (width 0.2) (layer "B.Cu") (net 44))
 (segment (start 173.355 120.015) (end 177.165 120.015) (width 0.2) (layer "B.Cu") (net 44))
 (segment (start 173.99 121.92) (end 172.085 120.015) (width 0.2) (layer "F.Cu") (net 22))
 (segment (start 172.085 120.015) (end 172.085 111.76) (width 0.2) (layer "F.Cu") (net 22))
 (segment (start 172.085 111.76) (end 170.165 109.84) (width 0.2) (layer "F.Cu") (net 22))
 (segment (start 176.53 121.92) (end 173.99 121.92) (width 0.2) (layer "F.Cu") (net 22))
 (segment (start 170.165 109.84) (end 165 109.84) (width 0.2) (layer "F.Cu") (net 22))
 (segment (start 154.94 89.42) (end 165 79.36) (width 0.2) (layer "B.Cu") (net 1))
 (segment (start 154.94 132.08) (end 154.94 89.42) (width 0.2) (layer "B.Cu") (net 1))
 (segment (start 135.129885 107.870115) (end 134.6 108.4) (width 0.2) (layer "F.Cu") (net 12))
 (segment (start 134.6 98.8) (end 135.653682 98.8) (width 0.2) (layer "F.Cu") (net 12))
 (segment (start 135.029885 101.970115) (end 134.8 102.2) (width 0.2) (layer "F.Cu") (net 12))
 (segment (start 135.873797 107.870115) (end 135.129885 107.870115) (width 0.2) (layer "F.Cu") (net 12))
 (segment (start 135.653682 98.8) (end 135.873797 99.020115) (width 0.2) (layer "F.Cu") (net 12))
 (segment (start 135.873797 101.970115) (end 135.029885 101.970115) (width 0.2) (layer "F.Cu") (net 12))
 (segment (start 135.873797 104.920115) (end 135.873797 101.970115) (width 0.2) (layer "F.Cu") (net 12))
 (via (at 134.8 102.2) (size 0.6) (drill 0.3) (layers "F.Cu" "B.Cu") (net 12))
 (via (at 134.6 108.4) (size 0.6) (drill 0.3) (layers "F.Cu" "B.Cu") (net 12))
 (via (at 134.6 98.8) (size 0.6) (drill 0.3) (layers "F.Cu" "B.Cu") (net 12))
 (segment (start 134 109.2) (end 134 103) (width 0.2) (layer "B.Cu") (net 12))
 (segment (start 134.6 124.4) (end 134 123.8) (width 0.2) (layer "B.Cu") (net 12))
 (segment (start 134 123.8) (end 134 109.2) (width 0.2) (layer "B.Cu") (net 12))
 (segment (start 134 109) (end 134 109.2) (width 0.2) (layer "B.Cu") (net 12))
 (segment (start 134.4 98.8) (end 134.6 98.8) (width 0.2) (layer "B.Cu") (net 12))
 (segment (start 134 103) (end 134 99.2) (width 0.2) (layer "B.Cu") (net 12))
 (segment (start 142.14 125.08) (end 135.28 125.08) (width 0.2) (layer "B.Cu") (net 12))
 (segment (start 135.28 125.08) (end 134.6 124.4) (width 0.2) (layer "B.Cu") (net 12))
 (segment (start 134 99.2) (end 134.4 98.8) (width 0.2) (layer "B.Cu") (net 12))
 (segment (start 134.6 108.4) (end 134 109) (width 0.2) (layer "B.Cu") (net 12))
 (segment (start 134.8 102.2) (end 134 103) (width 0.2) (layer "B.Cu") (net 12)))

